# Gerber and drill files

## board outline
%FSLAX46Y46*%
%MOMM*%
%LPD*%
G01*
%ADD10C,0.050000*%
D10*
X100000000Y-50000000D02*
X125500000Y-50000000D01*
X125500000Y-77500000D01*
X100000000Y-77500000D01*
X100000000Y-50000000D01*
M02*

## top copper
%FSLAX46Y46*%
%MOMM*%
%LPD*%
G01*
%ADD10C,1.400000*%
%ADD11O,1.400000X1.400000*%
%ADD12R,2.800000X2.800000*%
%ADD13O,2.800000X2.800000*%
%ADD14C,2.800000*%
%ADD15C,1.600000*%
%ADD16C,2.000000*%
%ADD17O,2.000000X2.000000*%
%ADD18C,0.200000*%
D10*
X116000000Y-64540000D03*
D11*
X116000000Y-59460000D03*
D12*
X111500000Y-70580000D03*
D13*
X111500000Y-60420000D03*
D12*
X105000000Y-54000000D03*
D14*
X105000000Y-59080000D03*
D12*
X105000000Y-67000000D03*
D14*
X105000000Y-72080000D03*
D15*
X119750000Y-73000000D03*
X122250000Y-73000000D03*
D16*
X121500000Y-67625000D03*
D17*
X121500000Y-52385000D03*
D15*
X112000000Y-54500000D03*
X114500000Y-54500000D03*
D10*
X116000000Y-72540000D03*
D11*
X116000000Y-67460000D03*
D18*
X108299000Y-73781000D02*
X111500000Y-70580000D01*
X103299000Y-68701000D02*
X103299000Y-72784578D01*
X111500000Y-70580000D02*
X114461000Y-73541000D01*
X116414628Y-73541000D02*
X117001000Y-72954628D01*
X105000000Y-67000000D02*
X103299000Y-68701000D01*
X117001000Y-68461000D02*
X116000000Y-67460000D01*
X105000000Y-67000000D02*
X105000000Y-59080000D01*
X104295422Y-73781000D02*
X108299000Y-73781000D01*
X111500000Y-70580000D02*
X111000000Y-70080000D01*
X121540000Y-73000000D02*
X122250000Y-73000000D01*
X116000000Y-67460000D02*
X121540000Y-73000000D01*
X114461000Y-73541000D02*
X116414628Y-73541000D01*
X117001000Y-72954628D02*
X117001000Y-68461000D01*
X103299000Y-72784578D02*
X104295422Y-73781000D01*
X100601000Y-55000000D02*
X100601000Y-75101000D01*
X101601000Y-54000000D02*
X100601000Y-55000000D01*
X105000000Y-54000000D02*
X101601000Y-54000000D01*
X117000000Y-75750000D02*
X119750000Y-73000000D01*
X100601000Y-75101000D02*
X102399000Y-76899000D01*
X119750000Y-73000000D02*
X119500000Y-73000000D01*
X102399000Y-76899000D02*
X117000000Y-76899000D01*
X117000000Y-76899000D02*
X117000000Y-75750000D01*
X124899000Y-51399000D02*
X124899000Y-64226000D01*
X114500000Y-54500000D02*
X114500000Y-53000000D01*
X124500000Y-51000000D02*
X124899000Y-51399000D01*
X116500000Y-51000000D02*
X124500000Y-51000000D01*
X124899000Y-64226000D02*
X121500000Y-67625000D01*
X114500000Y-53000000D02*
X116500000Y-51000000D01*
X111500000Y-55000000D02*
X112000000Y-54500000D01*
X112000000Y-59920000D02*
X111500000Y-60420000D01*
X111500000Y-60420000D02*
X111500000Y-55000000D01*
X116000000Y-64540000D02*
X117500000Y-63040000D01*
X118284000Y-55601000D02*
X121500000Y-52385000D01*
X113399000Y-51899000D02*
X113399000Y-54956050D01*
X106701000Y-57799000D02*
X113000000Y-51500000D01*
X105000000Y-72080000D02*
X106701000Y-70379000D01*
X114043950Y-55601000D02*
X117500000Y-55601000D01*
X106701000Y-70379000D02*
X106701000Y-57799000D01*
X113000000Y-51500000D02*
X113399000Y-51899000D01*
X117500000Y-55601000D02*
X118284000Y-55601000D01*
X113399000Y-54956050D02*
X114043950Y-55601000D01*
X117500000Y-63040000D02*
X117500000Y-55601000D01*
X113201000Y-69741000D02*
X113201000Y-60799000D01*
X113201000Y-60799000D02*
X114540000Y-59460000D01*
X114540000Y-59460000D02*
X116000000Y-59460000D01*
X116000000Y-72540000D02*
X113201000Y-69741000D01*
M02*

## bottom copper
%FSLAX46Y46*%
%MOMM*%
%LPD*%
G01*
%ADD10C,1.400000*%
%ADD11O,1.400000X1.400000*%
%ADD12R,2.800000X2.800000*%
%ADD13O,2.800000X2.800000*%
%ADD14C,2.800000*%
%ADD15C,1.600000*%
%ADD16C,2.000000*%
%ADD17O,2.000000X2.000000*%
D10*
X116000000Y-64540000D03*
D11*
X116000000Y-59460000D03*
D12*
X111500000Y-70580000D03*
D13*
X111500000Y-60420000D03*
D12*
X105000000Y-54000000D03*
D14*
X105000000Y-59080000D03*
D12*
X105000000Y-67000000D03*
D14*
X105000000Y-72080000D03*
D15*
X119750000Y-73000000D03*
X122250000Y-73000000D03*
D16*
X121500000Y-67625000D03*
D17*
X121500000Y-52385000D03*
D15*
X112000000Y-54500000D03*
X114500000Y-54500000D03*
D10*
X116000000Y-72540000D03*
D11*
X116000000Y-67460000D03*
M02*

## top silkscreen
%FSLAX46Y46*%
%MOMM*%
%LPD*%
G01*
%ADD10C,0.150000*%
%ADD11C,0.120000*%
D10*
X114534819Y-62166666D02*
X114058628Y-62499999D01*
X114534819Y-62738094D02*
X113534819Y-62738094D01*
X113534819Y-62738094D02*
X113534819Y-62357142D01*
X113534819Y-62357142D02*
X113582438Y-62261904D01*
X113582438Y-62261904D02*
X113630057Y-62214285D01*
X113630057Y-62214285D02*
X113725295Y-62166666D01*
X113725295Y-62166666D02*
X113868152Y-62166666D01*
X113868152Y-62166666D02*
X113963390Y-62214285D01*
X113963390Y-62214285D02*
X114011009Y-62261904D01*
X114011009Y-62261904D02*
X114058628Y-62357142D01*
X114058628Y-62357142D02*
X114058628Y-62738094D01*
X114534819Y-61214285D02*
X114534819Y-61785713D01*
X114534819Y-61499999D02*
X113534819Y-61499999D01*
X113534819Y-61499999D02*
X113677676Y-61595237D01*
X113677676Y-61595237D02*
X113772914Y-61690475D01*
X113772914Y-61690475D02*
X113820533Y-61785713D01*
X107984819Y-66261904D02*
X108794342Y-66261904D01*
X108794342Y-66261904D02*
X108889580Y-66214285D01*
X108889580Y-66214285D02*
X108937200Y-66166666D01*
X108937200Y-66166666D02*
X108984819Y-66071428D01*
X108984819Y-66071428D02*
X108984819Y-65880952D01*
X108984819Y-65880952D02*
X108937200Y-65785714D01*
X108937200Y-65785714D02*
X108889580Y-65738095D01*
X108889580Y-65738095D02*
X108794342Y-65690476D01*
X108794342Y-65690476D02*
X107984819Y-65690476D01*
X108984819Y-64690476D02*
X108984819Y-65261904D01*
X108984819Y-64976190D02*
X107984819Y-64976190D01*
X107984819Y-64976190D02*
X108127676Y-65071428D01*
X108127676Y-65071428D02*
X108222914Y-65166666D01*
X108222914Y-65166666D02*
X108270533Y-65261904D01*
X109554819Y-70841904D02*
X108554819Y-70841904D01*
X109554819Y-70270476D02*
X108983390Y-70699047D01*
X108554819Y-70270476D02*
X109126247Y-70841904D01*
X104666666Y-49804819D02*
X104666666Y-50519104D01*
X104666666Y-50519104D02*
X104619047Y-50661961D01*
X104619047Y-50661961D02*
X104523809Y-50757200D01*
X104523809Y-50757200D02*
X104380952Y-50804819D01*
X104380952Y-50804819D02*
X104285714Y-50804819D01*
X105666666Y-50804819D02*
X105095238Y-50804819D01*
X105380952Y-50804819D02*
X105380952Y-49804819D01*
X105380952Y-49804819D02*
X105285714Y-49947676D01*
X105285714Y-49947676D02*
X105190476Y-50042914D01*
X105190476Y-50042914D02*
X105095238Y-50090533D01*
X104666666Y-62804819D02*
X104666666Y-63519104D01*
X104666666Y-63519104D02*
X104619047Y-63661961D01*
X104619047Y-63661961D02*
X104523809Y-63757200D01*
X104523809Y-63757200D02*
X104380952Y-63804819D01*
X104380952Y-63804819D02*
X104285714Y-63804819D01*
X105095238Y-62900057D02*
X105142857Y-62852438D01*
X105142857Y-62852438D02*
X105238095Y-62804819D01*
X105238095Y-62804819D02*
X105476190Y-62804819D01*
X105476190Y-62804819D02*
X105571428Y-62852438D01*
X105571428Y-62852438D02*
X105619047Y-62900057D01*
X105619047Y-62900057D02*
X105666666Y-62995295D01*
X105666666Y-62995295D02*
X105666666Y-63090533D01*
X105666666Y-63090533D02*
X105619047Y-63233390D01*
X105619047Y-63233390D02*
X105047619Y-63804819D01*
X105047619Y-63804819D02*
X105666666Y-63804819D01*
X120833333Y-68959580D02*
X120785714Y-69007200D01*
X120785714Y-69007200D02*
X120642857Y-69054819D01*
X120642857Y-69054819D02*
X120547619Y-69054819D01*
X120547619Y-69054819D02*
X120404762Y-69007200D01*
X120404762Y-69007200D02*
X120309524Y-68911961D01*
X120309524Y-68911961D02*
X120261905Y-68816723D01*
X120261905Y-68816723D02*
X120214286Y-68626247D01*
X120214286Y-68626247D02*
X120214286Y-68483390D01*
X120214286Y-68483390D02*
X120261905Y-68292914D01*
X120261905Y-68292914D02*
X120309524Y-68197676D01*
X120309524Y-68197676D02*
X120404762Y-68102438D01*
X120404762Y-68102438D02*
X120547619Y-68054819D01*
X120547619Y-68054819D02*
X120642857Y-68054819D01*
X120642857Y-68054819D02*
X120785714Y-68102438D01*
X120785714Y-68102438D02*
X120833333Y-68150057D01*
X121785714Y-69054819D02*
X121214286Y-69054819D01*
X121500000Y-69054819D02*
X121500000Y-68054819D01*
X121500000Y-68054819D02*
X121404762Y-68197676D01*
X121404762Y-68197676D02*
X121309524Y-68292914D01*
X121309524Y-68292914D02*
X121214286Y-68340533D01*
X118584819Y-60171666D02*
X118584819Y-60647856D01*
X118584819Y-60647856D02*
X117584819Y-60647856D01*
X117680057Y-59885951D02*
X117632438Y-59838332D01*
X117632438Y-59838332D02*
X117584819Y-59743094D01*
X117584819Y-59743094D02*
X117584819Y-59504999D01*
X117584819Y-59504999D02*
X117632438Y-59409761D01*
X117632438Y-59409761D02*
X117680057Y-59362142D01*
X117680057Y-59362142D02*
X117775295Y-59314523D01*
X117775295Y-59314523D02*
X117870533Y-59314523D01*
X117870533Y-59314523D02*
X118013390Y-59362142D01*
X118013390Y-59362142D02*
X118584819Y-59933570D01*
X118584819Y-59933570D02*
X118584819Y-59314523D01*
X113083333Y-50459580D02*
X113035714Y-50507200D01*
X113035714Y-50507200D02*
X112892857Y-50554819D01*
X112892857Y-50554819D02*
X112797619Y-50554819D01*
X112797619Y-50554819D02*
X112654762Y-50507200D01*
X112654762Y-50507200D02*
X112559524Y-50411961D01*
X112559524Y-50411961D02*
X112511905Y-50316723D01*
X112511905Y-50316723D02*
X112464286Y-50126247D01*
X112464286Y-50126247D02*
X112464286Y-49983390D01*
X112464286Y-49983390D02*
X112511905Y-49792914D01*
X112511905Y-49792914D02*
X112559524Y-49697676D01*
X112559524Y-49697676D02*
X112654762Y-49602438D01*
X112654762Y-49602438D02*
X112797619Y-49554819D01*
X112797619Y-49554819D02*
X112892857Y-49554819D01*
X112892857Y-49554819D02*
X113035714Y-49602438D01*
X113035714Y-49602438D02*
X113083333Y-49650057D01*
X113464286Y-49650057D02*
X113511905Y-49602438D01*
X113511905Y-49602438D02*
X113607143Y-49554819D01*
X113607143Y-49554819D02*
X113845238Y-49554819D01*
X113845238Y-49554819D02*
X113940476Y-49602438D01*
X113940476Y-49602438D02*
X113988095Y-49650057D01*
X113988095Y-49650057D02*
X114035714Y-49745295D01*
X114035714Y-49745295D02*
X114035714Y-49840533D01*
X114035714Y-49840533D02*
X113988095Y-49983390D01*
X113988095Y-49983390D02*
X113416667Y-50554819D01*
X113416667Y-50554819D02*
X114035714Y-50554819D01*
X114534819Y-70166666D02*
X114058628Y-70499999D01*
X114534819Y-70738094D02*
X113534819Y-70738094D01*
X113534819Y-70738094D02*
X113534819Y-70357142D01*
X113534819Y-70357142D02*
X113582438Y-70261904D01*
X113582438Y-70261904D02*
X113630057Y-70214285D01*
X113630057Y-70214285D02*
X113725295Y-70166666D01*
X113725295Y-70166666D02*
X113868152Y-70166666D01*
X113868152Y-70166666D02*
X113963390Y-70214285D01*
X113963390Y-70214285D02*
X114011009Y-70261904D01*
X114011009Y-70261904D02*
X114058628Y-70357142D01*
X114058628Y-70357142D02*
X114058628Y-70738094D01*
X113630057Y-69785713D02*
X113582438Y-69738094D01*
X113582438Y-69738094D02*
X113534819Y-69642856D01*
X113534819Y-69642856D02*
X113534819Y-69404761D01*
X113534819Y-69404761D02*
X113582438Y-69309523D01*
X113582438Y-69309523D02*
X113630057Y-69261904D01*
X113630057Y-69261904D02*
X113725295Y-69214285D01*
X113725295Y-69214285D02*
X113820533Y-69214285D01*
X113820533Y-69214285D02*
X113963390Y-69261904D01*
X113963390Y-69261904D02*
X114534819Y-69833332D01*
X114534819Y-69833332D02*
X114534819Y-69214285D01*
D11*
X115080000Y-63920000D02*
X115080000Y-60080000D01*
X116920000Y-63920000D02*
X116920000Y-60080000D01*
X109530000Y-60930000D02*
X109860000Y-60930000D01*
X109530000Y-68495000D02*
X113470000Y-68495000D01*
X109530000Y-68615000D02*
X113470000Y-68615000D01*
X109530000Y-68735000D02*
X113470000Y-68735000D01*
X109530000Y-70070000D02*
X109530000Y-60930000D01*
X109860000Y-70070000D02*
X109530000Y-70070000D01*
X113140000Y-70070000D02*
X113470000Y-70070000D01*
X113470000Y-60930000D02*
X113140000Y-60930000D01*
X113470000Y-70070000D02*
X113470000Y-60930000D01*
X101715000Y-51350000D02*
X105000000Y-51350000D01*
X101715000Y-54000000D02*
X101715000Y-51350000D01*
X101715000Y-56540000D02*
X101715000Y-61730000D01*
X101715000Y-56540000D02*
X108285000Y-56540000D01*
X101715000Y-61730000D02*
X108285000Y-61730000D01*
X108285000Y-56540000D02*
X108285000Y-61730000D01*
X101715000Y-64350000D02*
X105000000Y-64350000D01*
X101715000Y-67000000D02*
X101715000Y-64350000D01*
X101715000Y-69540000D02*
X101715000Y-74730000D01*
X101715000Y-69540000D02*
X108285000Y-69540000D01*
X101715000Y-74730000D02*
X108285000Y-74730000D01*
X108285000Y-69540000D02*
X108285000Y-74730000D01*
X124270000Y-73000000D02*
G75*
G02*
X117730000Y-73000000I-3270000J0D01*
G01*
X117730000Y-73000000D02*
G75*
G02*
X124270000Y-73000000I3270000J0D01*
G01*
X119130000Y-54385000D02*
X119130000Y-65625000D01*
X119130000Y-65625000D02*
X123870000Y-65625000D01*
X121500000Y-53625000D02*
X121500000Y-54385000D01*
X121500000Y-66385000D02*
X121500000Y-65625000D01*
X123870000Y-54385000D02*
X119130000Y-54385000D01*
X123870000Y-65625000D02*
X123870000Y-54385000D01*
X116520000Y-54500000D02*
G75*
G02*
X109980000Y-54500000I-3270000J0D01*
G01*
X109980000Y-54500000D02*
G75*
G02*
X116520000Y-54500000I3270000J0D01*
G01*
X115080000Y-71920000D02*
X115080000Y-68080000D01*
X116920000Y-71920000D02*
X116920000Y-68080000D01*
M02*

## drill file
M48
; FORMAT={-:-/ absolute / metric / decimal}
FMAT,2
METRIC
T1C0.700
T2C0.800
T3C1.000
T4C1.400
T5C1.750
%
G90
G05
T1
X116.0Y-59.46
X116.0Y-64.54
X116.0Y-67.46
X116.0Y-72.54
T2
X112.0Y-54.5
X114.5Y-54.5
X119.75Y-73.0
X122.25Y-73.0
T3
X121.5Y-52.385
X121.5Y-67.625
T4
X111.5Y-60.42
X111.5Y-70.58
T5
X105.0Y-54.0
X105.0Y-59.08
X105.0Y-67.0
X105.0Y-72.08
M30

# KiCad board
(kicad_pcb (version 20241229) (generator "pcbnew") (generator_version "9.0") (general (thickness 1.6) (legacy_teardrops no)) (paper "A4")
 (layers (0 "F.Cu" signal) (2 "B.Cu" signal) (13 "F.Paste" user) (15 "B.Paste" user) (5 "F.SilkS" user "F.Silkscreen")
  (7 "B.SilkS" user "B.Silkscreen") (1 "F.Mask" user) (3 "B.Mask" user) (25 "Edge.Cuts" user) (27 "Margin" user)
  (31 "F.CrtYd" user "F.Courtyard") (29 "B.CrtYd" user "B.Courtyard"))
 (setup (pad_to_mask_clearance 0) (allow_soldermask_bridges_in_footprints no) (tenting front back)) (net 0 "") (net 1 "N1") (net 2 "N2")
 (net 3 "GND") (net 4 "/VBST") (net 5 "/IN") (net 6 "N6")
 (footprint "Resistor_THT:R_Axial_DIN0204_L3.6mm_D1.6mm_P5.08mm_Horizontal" (layer "F.Cu") (at 116 64.54 90)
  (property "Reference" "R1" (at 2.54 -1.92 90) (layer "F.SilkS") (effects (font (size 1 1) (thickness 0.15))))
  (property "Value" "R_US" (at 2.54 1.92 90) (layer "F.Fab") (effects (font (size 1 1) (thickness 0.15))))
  (fp_line (start 0.62 -0.92) (end 4.46 -0.92) (stroke (width 0.12) (type solid)) (layer "F.SilkS"))
  (fp_line (start 0.62 0.92) (end 4.46 0.92) (stroke (width 0.12) (type solid)) (layer "F.SilkS"))
  (pad "1" thru_hole circle (at 0 0 90) (size 1.4 1.4) (drill 0.7) (layers "*.Cu" "*.Mask") (remove_unused_layers no) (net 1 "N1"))
  (pad "2" thru_hole oval (at 5.08 0 90) (size 1.4 1.4) (drill 0.7) (layers "*.Cu" "*.Mask") (remove_unused_layers no) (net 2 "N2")))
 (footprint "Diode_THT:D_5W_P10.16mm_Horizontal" (layer "F.Cu") (at 111.5 70.58 90)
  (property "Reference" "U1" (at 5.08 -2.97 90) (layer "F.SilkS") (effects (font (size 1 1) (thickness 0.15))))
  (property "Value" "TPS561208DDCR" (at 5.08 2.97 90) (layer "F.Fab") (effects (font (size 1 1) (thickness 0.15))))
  (fp_line (start 9.65 -1.97) (end 9.65 -1.64) (stroke (width 0.12) (type solid)) (layer "F.SilkS"))
  (fp_line (start 2.085 -1.97) (end 2.085 1.97) (stroke (width 0.12) (type solid)) (layer "F.SilkS"))
  (fp_line (start 1.965 -1.97) (end 1.965 1.97) (stroke (width 0.12) (type solid)) (layer "F.SilkS"))
  (fp_line (start 1.845 -1.97) (end 1.845 1.97) (stroke (width 0.12) (type solid)) (layer "F.SilkS"))
  (fp_line (start 0.51 -1.97) (end 9.65 -1.97) (stroke (width 0.12) (type solid)) (layer "F.SilkS"))
  (fp_line (start 0.51 -1.64) (end 0.51 -1.97) (stroke (width 0.12) (type solid)) (layer "F.SilkS"))
  (fp_line (start 0.51 1.64) (end 0.51 1.97) (stroke (width 0.12) (type solid)) (layer "F.SilkS"))
  (fp_line (start 9.65 1.97) (end 9.65 1.64) (stroke (width 0.12) (type solid)) (layer "F.SilkS"))
  (fp_line (start 0.51 1.97) (end 9.65 1.97) (stroke (width 0.12) (type solid)) (layer "F.SilkS"))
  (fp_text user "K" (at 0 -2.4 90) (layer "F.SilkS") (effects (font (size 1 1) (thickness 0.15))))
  (pad "1" thru_hole rect (at 0 0 90) (size 2.8 2.8) (drill 1.4) (layers "*.Cu" "*.Mask") (remove_unused_layers no) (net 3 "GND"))
  (pad "2" thru_hole oval (at 10.16 0 90) (size 2.8 2.8) (drill 1.4) (layers "*.Cu" "*.Mask") (remove_unused_layers no) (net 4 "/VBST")))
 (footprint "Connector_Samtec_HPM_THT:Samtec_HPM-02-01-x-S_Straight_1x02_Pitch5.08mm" (layer "F.Cu") (at 105 54)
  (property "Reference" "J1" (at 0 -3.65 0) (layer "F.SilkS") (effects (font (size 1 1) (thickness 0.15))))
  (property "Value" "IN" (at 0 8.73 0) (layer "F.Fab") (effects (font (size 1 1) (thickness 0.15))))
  (fp_line (start -3.285 -2.65) (end 0 -2.65) (stroke (width 0.12) (type solid)) (layer "F.SilkS"))
  (fp_line (start -3.285 0) (end -3.285 -2.65) (stroke (width 0.12) (type solid)) (layer "F.SilkS"))
  (fp_line (start -3.285 2.54) (end -3.285 7.73) (stroke (width 0.12) (type solid)) (layer "F.SilkS"))
  (fp_line (start -3.285 2.54) (end 3.285 2.54) (stroke (width 0.12) (type solid)) (layer "F.SilkS"))
  (fp_line (start -3.285 7.73) (end 3.285 7.73) (stroke (width 0.12) (type solid)) (layer "F.SilkS"))
  (fp_line (start 3.285 2.54) (end 3.285 7.73) (stroke (width 0.12) (type solid)) (layer "F.SilkS"))
  (pad "1" thru_hole rect (at 0 0) (size 2.8 2.8) (drill 1.75) (layers "*.Cu" "*.Mask") (remove_unused_layers no) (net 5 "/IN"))
  (pad "2" thru_hole circle (at 0 5.08) (size 2.8 2.8) (drill 1.75) (layers "*.Cu" "*.Mask") (remove_unused_layers no) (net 3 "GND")))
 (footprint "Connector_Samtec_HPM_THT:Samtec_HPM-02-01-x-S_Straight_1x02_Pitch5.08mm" (layer "F.Cu") (at 105 67)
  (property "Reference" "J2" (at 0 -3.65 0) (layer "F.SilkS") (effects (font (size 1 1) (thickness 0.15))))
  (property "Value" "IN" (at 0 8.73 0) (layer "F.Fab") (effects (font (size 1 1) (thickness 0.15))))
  (fp_line (start -3.285 -2.65) (end 0 -2.65) (stroke (width 0.12) (type solid)) (layer "F.SilkS"))
  (fp_line (start -3.285 0) (end -3.285 -2.65) (stroke (width 0.12) (type solid)) (layer "F.SilkS"))
  (fp_line (start -3.285 2.54) (end -3.285 7.73) (stroke (width 0.12) (type solid)) (layer "F.SilkS"))
  (fp_line (start -3.285 2.54) (end 3.285 2.54) (stroke (width 0.12) (type solid)) (layer "F.SilkS"))
  (fp_line (start -3.285 7.73) (end 3.285 7.73) (stroke (width 0.12) (type solid)) (layer "F.SilkS"))
  (fp_line (start 3.285 2.54) (end 3.285 7.73) (stroke (width 0.12) (type solid)) (layer "F.SilkS"))
  (pad "1" thru_hole rect (at 0 0) (size 2.8 2.8) (drill 1.75) (layers "*.Cu" "*.Mask") (remove_unused_layers no) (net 3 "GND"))
  (pad "2" thru_hole circle (at 0 5.08) (size 2.8 2.8) (drill 1.75) (layers "*.Cu" "*.Mask") (remove_unused_layers no) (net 1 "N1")))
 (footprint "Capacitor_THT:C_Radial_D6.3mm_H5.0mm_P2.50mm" (layer "F.Cu") (at 119.75 73)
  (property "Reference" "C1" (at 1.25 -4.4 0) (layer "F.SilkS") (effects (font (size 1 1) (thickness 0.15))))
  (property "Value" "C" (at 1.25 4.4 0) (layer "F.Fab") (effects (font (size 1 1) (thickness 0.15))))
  (fp_circle (center 1.25 0) (end 4.52 0) (stroke (width 0.12) (type solid)) (fill no) (layer "F.SilkS"))
  (pad "1" thru_hole circle (at 0 0) (size 1.6 1.6) (drill 0.8) (layers "*.Cu" "*.Mask") (remove_unused_layers no) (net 5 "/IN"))
  (pad "2" thru_hole circle (at 2.5 0) (size 1.6 1.6) (drill 0.8) (layers "*.Cu" "*.Mask") (remove_unused_layers no) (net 3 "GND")))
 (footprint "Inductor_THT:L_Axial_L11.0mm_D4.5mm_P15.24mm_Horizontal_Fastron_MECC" (layer "F.Cu") (at 121.5 67.625 90)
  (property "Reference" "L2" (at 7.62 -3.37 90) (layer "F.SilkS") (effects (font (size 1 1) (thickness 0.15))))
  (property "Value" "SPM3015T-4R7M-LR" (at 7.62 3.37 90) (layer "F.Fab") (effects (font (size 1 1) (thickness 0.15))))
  (fp_line (start 13.24 -2.37) (end 2 -2.37) (stroke (width 0.12) (type solid)) (layer "F.SilkS"))
  (fp_line (start 2 -2.37) (end 2 2.37) (stroke (width 0.12) (type solid)) (layer "F.SilkS"))
  (fp_line (start 14 0) (end 13.24 0) (stroke (width 0.12) (type solid)) (layer "F.SilkS"))
  (fp_line (start 1.24 0) (end 2 0) (stroke (width 0.12) (type solid)) (layer "F.SilkS"))
  (fp_line (start 13.24 2.37) (end 13.24 -2.37) (stroke (width 0.12) (type solid)) (layer "F.SilkS"))
  (fp_line (start 2 2.37) (end 13.24 2.37) (stroke (width 0.12) (type solid)) (layer "F.SilkS"))
  (pad "1" thru_hole circle (at 0 0 90) (size 2 2) (drill 1) (layers "*.Cu" "*.Mask") (remove_unused_layers no) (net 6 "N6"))
  (pad "2" thru_hole oval (at 15.24 0 90) (size 2 2) (drill 1) (layers "*.Cu" "*.Mask") (remove_unused_layers no) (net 1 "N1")))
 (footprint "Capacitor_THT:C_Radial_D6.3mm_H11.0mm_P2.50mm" (layer "F.Cu") (at 112 54.5)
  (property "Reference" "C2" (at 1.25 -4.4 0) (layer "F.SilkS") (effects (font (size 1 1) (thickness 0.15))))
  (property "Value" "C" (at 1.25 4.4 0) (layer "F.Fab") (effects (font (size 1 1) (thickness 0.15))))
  (fp_circle (center 1.25 0) (end 4.52 0) (stroke (width 0.12) (type solid)) (fill no) (layer "F.SilkS"))
  (pad "1" thru_hole circle (at 0 0) (size 1.6 1.6) (drill 0.8) (layers "*.Cu" "*.Mask") (remove_unused_layers no) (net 4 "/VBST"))
  (pad "2" thru_hole circle (at 2.5 0) (size 1.6 1.6) (drill 0.8) (layers "*.Cu" "*.Mask") (remove_unused_layers no) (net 6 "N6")))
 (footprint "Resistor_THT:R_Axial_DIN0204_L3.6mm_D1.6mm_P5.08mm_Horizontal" (layer "F.Cu") (at 116 72.54 90)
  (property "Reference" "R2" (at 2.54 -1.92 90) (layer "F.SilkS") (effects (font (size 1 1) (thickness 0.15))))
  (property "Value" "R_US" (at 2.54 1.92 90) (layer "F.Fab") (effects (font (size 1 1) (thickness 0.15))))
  (fp_line (start 0.62 -0.92) (end 4.46 -0.92) (stroke (width 0.12) (type solid)) (layer "F.SilkS"))
  (fp_line (start 0.62 0.92) (end 4.46 0.92) (stroke (width 0.12) (type solid)) (layer "F.SilkS"))
  (pad "1" thru_hole circle (at 0 0 90) (size 1.4 1.4) (drill 0.7) (layers "*.Cu" "*.Mask") (remove_unused_layers no) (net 2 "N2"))
  (pad "2" thru_hole oval (at 5.08 0 90) (size 1.4 1.4) (drill 0.7) (layers "*.Cu" "*.Mask") (remove_unused_layers no) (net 3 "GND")))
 (gr_rect (start 100 50) (end 125.5 77.5) (stroke (width 0.05) (type default)) (fill no) (layer "Edge.Cuts"))
 (segment (start 108.299 73.781) (end 111.5 70.58) (width 0.2) (layer "F.Cu") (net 3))
 (segment (start 103.299 68.701) (end 103.299 72.784578) (width 0.2) (layer "F.Cu") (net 3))
 (segment (start 111.5 70.58) (end 114.461 73.541) (width 0.2) (layer "F.Cu") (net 3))
 (segment (start 116.414628 73.541) (end 117.001 72.954628) (width 0.2) (layer "F.Cu") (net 3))
 (segment (start 105 67) (end 103.299 68.701) (width 0.2) (layer "F.Cu") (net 3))
 (segment (start 117.001 68.461) (end 116 67.46) (width 0.2) (layer "F.Cu") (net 3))
 (segment (start 105 67) (end 105 59.08) (width 0.2) (layer "F.Cu") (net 3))
 (segment (start 104.295422 73.781) (end 108.299 73.781) (width 0.2) (layer "F.Cu") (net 3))
 (segment (start 111.5 70.58) (end 111 70.08) (width 0.2) (layer "F.Cu") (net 3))
 (segment (start 121.54 73) (end 122.25 73) (width 0.2) (layer "F.Cu") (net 3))
 (segment (start 116 67.46) (end 121.54 73) (width 0.2) (layer "F.Cu") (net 3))
 (segment (start 114.461 73.541) (end 116.414628 73.541) (width 0.2) (layer "F.Cu") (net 3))
 (segment (start 117.001 72.954628) (end 117.001 68.461) (width 0.2) (layer "F.Cu") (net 3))
 (segment (start 103.299 72.784578) (end 104.295422 73.781) (width 0.2) (layer "F.Cu") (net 3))
 (segment (start 100.601 55) (end 100.601 75.101) (width 0.2) (layer "F.Cu") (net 5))
 (segment (start 101.601 54) (end 100.601 55) (width 0.2) (layer "F.Cu") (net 5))
 (segment (start 105 54) (end 101.601 54) (width 0.2) (layer "F.Cu") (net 5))
 (segment (start 117 75.75) (end 119.75 73) (width 0.2) (layer "F.Cu") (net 5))
 (segment (start 100.601 75.101) (end 102.399 76.899) (width 0.2) (layer "F.Cu") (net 5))
 (segment (start 119.75 73) (end 119.5 73) (width 0.2) (layer "F.Cu") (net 5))
 (segment (start 102.399 76.899) (end 117 76.899) (width 0.2) (layer "F.Cu") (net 5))
 (segment (start 117 76.899) (end 117 75.75) (width 0.2) (layer "F.Cu") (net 5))
 (segment (start 124.899 51.399) (end 124.899 64.226) (width 0.2) (layer "F.Cu") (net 6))
 (segment (start 114.5 54.5) (end 114.5 53) (width 0.2) (layer "F.Cu") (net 6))
 (segment (start 124.5 51) (end 124.899 51.399) (width 0.2) (layer "F.Cu") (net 6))
 (segment (start 116.5 51) (end 124.5 51) (width 0.2) (layer "F.Cu") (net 6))
 (segment (start 124.899 64.226) (end 121.5 67.625) (width 0.2) (layer "F.Cu") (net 6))
 (segment (start 114.5 53) (end 116.5 51) (width 0.2) (layer "F.Cu") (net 6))
 (segment (start 111.5 55) (end 112 54.5) (width 0.2) (layer "F.Cu") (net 4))
 (segment (start 112 59.92) (end 111.5 60.42) (width 0.2) (layer "F.Cu") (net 4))
 (segment (start 111.5 60.42) (end 111.5 55) (width 0.2) (layer "F.Cu") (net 4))
 (segment (start 116 64.54) (end 117.5 63.04) (width 0.2) (layer "F.Cu") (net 1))
 (segment (start 118.284 55.601) (end 121.5 52.385) (width 0.2) (layer "F.Cu") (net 1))
 (segment (start 113.399 51.899) (end 113.399 54.95605) (width 0.2) (layer "F.Cu") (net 1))
 (segment (start 106.701 57.799) (end 113 51.5) (width 0.2) (layer "F.Cu") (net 1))
 (segment (start 105 72.08) (end 106.701 70.379) (width 0.2) (layer "F.Cu") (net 1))
 (segment (start 114.04395 55.601) (end 117.5 55.601) (width 0.2) (layer "F.Cu") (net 1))
 (segment (start 106.701 70.379) (end 106.701 57.799) (width 0.2) (layer "F.Cu") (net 1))
 (segment (start 113 51.5) (end 113.399 51.899) (width 0.2) (layer "F.Cu") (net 1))
 (segment (start 117.5 55.601) (end 118.284 55.601) (width 0.2) (layer "F.Cu") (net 1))
 (segment (start 113.399 54.95605) (end 114.04395 55.601) (width 0.2) (layer "F.Cu") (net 1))
 (segment (start 117.5 63.04) (end 117.5 55.601) (width 0.2) (layer "F.Cu") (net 1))
 (segment (start 113.201 69.741) (end 113.201 60.799) (width 0.2) (layer "F.Cu") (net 2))
 (segment (start 113.201 60.799) (end 114.54 59.46) (width 0.2) (layer "F.Cu") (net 2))
 (segment (start 114.54 59.46) (end 116 59.46) (width 0.2) (layer "F.Cu") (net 2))
 (segment (start 116 72.54) (end 113.201 69.741) (width 0.2) (layer "F.Cu") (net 2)))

